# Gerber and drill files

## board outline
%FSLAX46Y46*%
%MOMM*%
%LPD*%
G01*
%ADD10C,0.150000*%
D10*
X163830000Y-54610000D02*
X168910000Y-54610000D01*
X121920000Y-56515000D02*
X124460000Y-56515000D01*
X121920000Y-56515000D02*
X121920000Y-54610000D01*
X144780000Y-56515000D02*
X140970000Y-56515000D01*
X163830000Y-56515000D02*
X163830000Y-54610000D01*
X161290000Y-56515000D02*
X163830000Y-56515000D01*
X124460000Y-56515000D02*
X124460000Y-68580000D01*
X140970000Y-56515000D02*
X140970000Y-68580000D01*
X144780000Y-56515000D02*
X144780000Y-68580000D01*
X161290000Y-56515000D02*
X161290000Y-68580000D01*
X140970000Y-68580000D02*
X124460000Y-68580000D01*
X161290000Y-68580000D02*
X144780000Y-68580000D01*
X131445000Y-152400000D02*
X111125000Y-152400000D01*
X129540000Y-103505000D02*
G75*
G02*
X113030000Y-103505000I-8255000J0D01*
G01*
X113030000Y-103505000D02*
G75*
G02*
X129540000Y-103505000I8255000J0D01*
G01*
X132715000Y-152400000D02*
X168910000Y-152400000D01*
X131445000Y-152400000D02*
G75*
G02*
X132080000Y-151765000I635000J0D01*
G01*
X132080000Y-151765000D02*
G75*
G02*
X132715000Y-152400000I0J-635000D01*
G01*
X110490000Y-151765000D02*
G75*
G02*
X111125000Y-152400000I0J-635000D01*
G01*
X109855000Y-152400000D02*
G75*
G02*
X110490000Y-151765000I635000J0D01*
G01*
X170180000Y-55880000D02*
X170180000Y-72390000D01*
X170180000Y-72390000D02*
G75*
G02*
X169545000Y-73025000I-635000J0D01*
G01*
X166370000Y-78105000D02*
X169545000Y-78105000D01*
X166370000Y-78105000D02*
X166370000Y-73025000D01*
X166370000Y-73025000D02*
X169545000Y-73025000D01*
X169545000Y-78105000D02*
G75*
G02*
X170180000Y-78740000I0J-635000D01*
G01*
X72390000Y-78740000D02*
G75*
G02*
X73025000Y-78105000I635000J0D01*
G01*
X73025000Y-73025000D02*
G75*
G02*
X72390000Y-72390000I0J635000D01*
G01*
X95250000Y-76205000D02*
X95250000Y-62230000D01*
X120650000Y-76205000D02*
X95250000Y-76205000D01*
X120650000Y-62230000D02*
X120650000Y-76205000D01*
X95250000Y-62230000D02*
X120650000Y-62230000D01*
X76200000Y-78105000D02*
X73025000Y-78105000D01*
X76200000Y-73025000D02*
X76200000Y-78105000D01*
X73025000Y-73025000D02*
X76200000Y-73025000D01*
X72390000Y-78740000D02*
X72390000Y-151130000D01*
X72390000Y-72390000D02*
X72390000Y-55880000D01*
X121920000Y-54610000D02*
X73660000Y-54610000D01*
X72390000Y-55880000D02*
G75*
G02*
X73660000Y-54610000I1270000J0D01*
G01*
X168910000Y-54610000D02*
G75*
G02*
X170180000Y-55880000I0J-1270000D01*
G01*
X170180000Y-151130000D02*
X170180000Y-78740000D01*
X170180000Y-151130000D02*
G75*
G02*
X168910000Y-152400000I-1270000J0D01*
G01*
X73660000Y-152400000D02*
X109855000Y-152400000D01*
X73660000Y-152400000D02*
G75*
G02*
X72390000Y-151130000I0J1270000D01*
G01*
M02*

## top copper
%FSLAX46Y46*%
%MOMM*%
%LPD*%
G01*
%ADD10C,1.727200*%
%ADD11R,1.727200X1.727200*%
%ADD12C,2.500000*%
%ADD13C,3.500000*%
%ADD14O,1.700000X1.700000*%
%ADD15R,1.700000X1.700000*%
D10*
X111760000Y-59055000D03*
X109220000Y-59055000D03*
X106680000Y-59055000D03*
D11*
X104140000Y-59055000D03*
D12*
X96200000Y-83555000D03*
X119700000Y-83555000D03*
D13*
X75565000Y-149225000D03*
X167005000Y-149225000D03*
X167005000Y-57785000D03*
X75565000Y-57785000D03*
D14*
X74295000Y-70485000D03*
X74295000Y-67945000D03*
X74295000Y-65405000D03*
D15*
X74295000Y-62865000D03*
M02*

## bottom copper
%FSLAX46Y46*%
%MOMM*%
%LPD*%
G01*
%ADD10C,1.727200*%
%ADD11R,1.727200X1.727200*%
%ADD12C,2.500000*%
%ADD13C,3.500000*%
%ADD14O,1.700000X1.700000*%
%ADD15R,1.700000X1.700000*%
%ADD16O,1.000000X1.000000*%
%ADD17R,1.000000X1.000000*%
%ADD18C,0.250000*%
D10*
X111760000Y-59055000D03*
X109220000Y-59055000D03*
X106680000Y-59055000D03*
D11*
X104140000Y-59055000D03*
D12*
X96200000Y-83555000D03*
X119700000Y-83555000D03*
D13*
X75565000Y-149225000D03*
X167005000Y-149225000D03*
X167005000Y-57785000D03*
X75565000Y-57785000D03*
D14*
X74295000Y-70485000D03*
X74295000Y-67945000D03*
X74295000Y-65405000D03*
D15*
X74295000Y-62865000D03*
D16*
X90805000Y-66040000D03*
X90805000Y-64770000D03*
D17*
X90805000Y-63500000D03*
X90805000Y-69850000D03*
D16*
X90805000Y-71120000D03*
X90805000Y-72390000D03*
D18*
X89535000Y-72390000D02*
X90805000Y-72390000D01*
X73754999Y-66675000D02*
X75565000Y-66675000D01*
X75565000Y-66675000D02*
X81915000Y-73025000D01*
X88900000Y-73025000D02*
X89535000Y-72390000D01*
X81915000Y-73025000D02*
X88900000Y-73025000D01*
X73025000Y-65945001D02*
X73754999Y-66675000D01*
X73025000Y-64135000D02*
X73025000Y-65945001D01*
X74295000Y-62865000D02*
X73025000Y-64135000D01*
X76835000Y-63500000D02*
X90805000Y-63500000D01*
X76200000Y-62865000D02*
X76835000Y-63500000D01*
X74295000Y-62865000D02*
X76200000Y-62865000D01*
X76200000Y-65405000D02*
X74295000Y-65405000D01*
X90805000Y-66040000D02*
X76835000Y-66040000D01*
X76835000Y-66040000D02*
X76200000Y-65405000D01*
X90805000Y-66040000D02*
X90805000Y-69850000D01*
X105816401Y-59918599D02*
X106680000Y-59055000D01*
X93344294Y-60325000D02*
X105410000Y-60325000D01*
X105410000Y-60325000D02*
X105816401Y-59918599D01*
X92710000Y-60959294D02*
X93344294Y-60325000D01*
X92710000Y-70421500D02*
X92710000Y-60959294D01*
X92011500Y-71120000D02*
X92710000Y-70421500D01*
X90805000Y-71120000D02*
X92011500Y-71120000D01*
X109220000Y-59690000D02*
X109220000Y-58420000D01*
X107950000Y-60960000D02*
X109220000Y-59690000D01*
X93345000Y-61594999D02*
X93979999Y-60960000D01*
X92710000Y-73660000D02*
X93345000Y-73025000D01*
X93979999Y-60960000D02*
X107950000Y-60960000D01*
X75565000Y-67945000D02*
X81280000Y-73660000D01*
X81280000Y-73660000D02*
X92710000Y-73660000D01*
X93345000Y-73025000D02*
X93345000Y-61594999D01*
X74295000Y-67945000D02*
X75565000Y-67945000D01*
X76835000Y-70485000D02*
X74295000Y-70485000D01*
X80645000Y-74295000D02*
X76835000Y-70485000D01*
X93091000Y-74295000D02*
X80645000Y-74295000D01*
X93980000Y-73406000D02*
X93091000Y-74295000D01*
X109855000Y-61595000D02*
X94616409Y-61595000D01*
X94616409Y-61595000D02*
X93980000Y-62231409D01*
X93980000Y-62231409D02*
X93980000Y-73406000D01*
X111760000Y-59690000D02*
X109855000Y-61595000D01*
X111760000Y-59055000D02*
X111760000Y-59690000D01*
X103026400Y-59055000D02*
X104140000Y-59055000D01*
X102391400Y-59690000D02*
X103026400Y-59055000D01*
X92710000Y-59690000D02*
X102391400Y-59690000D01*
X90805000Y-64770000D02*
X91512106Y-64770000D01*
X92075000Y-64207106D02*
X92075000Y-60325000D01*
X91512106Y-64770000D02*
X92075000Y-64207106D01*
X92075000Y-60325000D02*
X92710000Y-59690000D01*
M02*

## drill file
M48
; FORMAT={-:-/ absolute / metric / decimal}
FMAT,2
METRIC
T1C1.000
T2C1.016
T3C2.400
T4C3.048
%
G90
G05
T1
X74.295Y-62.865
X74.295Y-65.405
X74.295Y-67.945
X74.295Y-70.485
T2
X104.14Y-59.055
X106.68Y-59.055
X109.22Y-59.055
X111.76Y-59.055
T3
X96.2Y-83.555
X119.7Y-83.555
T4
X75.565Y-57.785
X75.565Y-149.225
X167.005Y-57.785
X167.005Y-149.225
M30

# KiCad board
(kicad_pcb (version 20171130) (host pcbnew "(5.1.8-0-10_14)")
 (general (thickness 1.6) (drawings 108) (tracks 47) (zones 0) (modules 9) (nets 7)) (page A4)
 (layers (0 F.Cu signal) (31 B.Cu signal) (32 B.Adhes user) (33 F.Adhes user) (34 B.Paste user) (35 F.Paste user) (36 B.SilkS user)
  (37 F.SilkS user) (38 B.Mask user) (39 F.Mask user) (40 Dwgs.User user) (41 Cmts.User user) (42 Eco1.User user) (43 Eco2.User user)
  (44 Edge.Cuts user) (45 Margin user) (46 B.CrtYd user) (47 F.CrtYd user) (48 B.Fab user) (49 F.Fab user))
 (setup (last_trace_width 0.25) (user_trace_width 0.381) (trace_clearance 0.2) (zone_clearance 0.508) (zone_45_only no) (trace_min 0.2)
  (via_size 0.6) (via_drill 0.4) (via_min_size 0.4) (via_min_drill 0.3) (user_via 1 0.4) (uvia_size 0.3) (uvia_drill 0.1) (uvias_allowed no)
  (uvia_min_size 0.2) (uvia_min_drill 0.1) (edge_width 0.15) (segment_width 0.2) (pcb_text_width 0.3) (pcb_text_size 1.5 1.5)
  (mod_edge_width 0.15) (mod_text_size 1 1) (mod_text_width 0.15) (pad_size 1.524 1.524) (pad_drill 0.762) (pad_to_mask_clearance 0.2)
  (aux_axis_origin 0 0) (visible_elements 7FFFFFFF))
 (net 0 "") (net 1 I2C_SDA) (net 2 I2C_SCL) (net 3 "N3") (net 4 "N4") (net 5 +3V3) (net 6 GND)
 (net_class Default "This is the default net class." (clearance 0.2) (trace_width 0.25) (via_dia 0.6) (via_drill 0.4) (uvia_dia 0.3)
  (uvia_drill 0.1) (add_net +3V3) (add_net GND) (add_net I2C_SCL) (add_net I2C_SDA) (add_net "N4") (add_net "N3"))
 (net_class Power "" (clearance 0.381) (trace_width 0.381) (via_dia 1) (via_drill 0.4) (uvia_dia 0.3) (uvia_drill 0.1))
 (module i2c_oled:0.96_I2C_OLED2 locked (layer F.Cu) (at 107.95 59.055)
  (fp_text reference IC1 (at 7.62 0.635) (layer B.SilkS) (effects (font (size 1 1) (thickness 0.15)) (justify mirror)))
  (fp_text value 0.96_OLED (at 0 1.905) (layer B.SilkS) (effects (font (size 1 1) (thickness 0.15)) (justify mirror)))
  (pad 4 thru_hole circle (at 3.81 0) (size 1.7272 1.7272) (drill 1.016) (layers *.Cu *.Mask) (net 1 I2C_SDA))
  (pad 3 thru_hole circle (at 1.27 0) (size 1.7272 1.7272) (drill 1.016) (layers *.Cu *.Mask) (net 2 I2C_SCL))
  (pad 2 thru_hole circle (at -1.27 0) (size 1.7272 1.7272) (drill 1.016) (layers *.Cu *.Mask) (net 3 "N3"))
  (pad 1 thru_hole rect (at -3.81 0) (size 1.7272 1.7272) (drill 1.016) (layers *.Cu *.Mask) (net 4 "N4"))
  (pad "" np_thru_hole circle (at -11.75 24.5) (size 2.5 2.5) (drill 2.4) (layers *.Cu *.Mask))
  (pad "" np_thru_hole circle (at 11.75 24.5) (size 2.5 2.5) (drill 2.4) (layers *.Cu *.Mask)))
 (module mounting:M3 (layer F.Cu) (at 75.565 149.225)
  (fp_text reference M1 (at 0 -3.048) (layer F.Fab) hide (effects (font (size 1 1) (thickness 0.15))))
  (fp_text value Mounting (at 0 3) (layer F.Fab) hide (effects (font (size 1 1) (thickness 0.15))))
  (pad "" np_thru_hole circle (at 0 0) (size 3.5 3.5) (drill 3.048) (layers *.Cu *.Mask) (solder_mask_margin 0.8)))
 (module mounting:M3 (layer F.Cu) (at 167.005 149.225)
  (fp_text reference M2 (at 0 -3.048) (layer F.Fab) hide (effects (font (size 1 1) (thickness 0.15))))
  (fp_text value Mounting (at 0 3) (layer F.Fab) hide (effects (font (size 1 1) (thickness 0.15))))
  (pad "" np_thru_hole circle (at 0 0) (size 3.5 3.5) (drill 3.048) (layers *.Cu *.Mask) (solder_mask_margin 0.8)))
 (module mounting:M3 (layer F.Cu) (at 167.005 57.785)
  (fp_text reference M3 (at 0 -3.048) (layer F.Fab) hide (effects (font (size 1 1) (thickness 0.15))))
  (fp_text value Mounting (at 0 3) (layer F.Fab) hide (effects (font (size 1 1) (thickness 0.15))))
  (pad "" np_thru_hole circle (at 0 0) (size 3.5 3.5) (drill 3.048) (layers *.Cu *.Mask) (solder_mask_margin 0.8)))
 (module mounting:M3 (layer F.Cu) (at 75.565 57.785)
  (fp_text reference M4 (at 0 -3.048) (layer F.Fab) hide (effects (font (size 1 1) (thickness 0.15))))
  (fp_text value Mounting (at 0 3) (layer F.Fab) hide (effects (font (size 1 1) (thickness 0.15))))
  (pad "" np_thru_hole circle (at 0 0) (size 3.5 3.5) (drill 3.048) (layers *.Cu *.Mask) (solder_mask_margin 0.8)))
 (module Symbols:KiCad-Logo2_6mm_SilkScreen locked (layer B.Cu) (at 142.875 88.9 180)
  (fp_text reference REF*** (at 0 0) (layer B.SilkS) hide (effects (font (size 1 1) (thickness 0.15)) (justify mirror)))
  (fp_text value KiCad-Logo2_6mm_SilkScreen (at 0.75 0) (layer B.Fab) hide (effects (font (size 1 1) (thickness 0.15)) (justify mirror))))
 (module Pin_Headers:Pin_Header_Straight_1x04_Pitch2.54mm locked (layer B.Cu) (at 74.295 62.865 180)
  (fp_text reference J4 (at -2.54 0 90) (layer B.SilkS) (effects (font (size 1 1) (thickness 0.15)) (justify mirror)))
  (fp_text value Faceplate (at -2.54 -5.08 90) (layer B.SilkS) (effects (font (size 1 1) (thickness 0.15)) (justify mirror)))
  (pad 4 thru_hole oval (at 0 -7.62 180) (size 1.7 1.7) (drill 1) (layers *.Cu *.Mask) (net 1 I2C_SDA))
  (pad 3 thru_hole oval (at 0 -5.08 180) (size 1.7 1.7) (drill 1) (layers *.Cu *.Mask) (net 2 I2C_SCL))
  (pad 2 thru_hole oval (at 0 -2.54 180) (size 1.7 1.7) (drill 1) (layers *.Cu *.Mask) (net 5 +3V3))
  (pad 1 thru_hole rect (at 0 0 180) (size 1.7 1.7) (drill 1) (layers *.Cu *.Mask) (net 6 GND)))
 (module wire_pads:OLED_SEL (layer B.Cu) (at 90.805 63.5 180)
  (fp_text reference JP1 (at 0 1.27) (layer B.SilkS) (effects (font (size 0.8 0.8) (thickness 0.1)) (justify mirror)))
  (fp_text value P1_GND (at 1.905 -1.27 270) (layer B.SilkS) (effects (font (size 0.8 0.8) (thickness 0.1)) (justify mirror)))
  (pad 3 smd oval (at 0 -2.54 180) (size 1 1) (layers B.Cu B.Paste B.Mask) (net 5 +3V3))
  (pad 2 smd oval (at 0 -1.27 180) (size 1 1) (layers B.Cu B.Paste B.Mask) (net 4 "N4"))
  (pad 1 smd rect (at 0 0 180) (size 1 1) (layers B.Cu B.Paste B.Mask) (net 6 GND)))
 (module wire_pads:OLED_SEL (layer B.Cu) (at 90.805 69.85 180)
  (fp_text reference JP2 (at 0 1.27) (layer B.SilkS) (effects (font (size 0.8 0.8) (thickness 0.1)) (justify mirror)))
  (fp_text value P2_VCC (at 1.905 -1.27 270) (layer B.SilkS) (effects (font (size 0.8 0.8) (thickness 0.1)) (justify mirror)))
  (pad 1 smd rect (at 0 0 180) (size 1 1) (layers B.Cu B.Paste B.Mask) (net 5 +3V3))
  (pad 2 smd oval (at 0 -1.27 180) (size 1 1) (layers B.Cu B.Paste B.Mask) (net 3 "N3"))
  (pad 3 smd oval (at 0 -2.54 180) (size 1 1) (layers B.Cu B.Paste B.Mask) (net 6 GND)))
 (gr_line (start 163.83 54.61) (end 168.91 54.61) (layer Edge.Cuts) (width 0.15))
 (gr_line (start 121.92 56.515) (end 124.46 56.515) (layer Edge.Cuts) (width 0.15))
 (gr_line (start 121.92 56.515) (end 121.92 54.61) (layer Edge.Cuts) (width 0.15))
 (gr_line (start 144.78 56.515) (end 140.97 56.515) (layer Edge.Cuts) (width 0.15))
 (gr_line (start 163.83 56.515) (end 163.83 54.61) (layer Edge.Cuts) (width 0.15))
 (gr_line (start 161.29 56.515) (end 163.83 56.515) (layer Edge.Cuts) (width 0.15))
 (gr_line (start 124.46 56.515) (end 124.46 68.58) (layer Edge.Cuts) (width 0.15))
 (gr_line (start 140.97 56.515) (end 140.97 68.58) (layer Edge.Cuts) (width 0.15))
 (gr_line (start 144.78 56.515) (end 144.78 68.58) (layer Edge.Cuts) (width 0.15))
 (gr_line (start 161.29 56.515) (end 161.29 68.58) (layer Edge.Cuts) (width 0.15))
 (gr_line (start 140.97 68.58) (end 124.46 68.58) (layer Edge.Cuts) (width 0.15))
 (gr_line (start 161.29 68.58) (end 144.78 68.58) (layer Edge.Cuts) (width 0.15))
 (gr_line (start 131.445 152.4) (end 111.125 152.4) (layer Edge.Cuts) (width 0.15))
 (gr_circle (center 121.285 103.505) (end 129.54 103.505) (layer Edge.Cuts) (width 0.15))
 (gr_line (start 132.715 152.4) (end 168.91 152.4) (layer Edge.Cuts) (width 0.15))
 (gr_arc (start 132.08 152.4) (end 132.08 151.765) (angle -90) (layer Edge.Cuts) (width 0.15))
 (gr_arc (start 132.08 152.4) (end 132.715 152.4) (angle -90) (layer Edge.Cuts) (width 0.15))
 (gr_arc (start 110.49 152.4) (end 111.125 152.4) (angle -90) (layer Edge.Cuts) (width 0.15))
 (gr_arc (start 110.49 152.4) (end 110.49 151.765) (angle -90) (layer Edge.Cuts) (width 0.15))
 (gr_line (start 170.18 55.88) (end 170.18 72.39) (layer Edge.Cuts) (width 0.15))
 (gr_arc (start 169.545 72.39) (end 169.545 73.025) (angle -90) (layer Edge.Cuts) (width 0.15))
 (gr_line (start 166.37 78.105) (end 169.545 78.105) (layer Edge.Cuts) (width 0.15))
 (gr_line (start 166.37 78.105) (end 166.37 73.025) (layer Edge.Cuts) (width 0.15))
 (gr_line (start 166.37 73.025) (end 169.545 73.025) (layer Edge.Cuts) (width 0.15))
 (gr_arc (start 169.545 78.74) (end 170.18 78.74) (angle -90) (layer Edge.Cuts) (width 0.15))
 (gr_arc (start 73.025 78.74) (end 73.025 78.105) (angle -90) (layer Edge.Cuts) (width 0.15))
 (gr_arc (start 73.025 72.39) (end 72.39 72.39) (angle -90) (layer Edge.Cuts) (width 0.15))
 (gr_line (start 95.25 76.205) (end 95.25 62.23) (layer Edge.Cuts) (width 0.15))
 (gr_line (start 120.65 76.205) (end 95.25 76.205) (layer Edge.Cuts) (width 0.15))
 (gr_line (start 120.65 62.23) (end 120.65 76.205) (layer Edge.Cuts) (width 0.15))
 (gr_line (start 95.25 62.23) (end 120.65 62.23) (layer Edge.Cuts) (width 0.15))
 (gr_line (start 76.2 78.105) (end 73.025 78.105) (layer Edge.Cuts) (width 0.15))
 (gr_line (start 76.2 73.025) (end 76.2 78.105) (layer Edge.Cuts) (width 0.15))
 (gr_line (start 73.025 73.025) (end 76.2 73.025) (layer Edge.Cuts) (width 0.15))
 (gr_line (start 72.39 78.74) (end 72.39 151.13) (layer Edge.Cuts) (width 0.15))
 (gr_line (start 72.39 72.39) (end 72.39 55.88) (layer Edge.Cuts) (width 0.15))
 (gr_line (start 121.92 54.61) (end 73.66 54.61) (angle 90) (layer Edge.Cuts) (width 0.15))
 (gr_arc (start 73.66 55.88) (end 72.39 55.88) (angle 90) (layer Edge.Cuts) (width 0.15))
 (gr_arc (start 168.91 55.88) (end 168.91 54.61) (angle 90) (layer Edge.Cuts) (width 0.15))
 (gr_line (start 170.18 151.13) (end 170.18 78.74) (angle 90) (layer Edge.Cuts) (width 0.15))
 (gr_arc (start 168.91 151.13) (end 170.18 151.13) (angle 90) (layer Edge.Cuts) (width 0.15))
 (gr_line (start 73.66 152.4) (end 109.855 152.4) (angle 90) (layer Edge.Cuts) (width 0.15))
 (gr_arc (start 73.66 151.13) (end 73.66 152.4) (angle 90) (layer Edge.Cuts) (width 0.15))
 (segment (start 89.535 72.39) (end 90.805 72.39) (width 0.25) (layer B.Cu) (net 6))
 (segment (start 73.754999 66.675) (end 75.565 66.675) (width 0.25) (layer B.Cu) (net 6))
 (segment (start 75.565 66.675) (end 81.915 73.025) (width 0.25) (layer B.Cu) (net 6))
 (segment (start 88.9 73.025) (end 89.535 72.39) (width 0.25) (layer B.Cu) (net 6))
 (segment (start 81.915 73.025) (end 88.9 73.025) (width 0.25) (layer B.Cu) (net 6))
 (segment (start 73.025 65.945001) (end 73.754999 66.675) (width 0.25) (layer B.Cu) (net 6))
 (segment (start 73.025 64.135) (end 73.025 65.945001) (width 0.25) (layer B.Cu) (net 6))
 (segment (start 74.295 62.865) (end 73.025 64.135) (width 0.25) (layer B.Cu) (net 6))
 (segment (start 76.835 63.5) (end 90.805 63.5) (width 0.25) (layer B.Cu) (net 6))
 (segment (start 76.2 62.865) (end 76.835 63.5) (width 0.25) (layer B.Cu) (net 6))
 (segment (start 74.295 62.865) (end 76.2 62.865) (width 0.25) (layer B.Cu) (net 6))
 (segment (start 76.2 65.405) (end 74.295 65.405) (width 0.25) (layer B.Cu) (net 5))
 (segment (start 90.805 66.04) (end 76.835 66.04) (width 0.25) (layer B.Cu) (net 5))
 (segment (start 76.835 66.04) (end 76.2 65.405) (width 0.25) (layer B.Cu) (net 5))
 (segment (start 90.805 66.04) (end 90.805 69.85) (width 0.25) (layer B.Cu) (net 5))
 (segment (start 105.816401 59.918599) (end 106.68 59.055) (width 0.25) (layer B.Cu) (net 3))
 (segment (start 93.344294 60.325) (end 105.41 60.325) (width 0.25) (layer B.Cu) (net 3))
 (segment (start 105.41 60.325) (end 105.816401 59.918599) (width 0.25) (layer B.Cu) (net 3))
 (segment (start 92.71 60.959294) (end 93.344294 60.325) (width 0.25) (layer B.Cu) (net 3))
 (segment (start 92.71 70.4215) (end 92.71 60.959294) (width 0.25) (layer B.Cu) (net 3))
 (segment (start 92.0115 71.12) (end 92.71 70.4215) (width 0.25) (layer B.Cu) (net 3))
 (segment (start 90.805 71.12) (end 92.0115 71.12) (width 0.25) (layer B.Cu) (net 3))
 (segment (start 109.22 59.69) (end 109.22 58.42) (width 0.25) (layer B.Cu) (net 2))
 (segment (start 107.95 60.96) (end 109.22 59.69) (width 0.25) (layer B.Cu) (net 2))
 (segment (start 93.345 61.594999) (end 93.979999 60.96) (width 0.25) (layer B.Cu) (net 2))
 (segment (start 92.71 73.66) (end 93.345 73.025) (width 0.25) (layer B.Cu) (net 2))
 (segment (start 93.979999 60.96) (end 107.95 60.96) (width 0.25) (layer B.Cu) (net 2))
 (segment (start 75.565 67.945) (end 81.28 73.66) (width 0.25) (layer B.Cu) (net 2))
 (segment (start 81.28 73.66) (end 92.71 73.66) (width 0.25) (layer B.Cu) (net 2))
 (segment (start 93.345 73.025) (end 93.345 61.594999) (width 0.25) (layer B.Cu) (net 2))
 (segment (start 74.295 67.945) (end 75.565 67.945) (width 0.25) (layer B.Cu) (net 2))
 (segment (start 76.835 70.485) (end 74.295 70.485) (width 0.25) (layer B.Cu) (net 1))
 (segment (start 80.645 74.295) (end 76.835 70.485) (width 0.25) (layer B.Cu) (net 1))
 (segment (start 93.091 74.295) (end 80.645 74.295) (width 0.25) (layer B.Cu) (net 1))
 (segment (start 93.98 73.406) (end 93.091 74.295) (width 0.25) (layer B.Cu) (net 1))
 (segment (start 109.855 61.595) (end 94.616409 61.595) (width 0.25) (layer B.Cu) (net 1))
 (segment (start 94.616409 61.595) (end 93.98 62.231409) (width 0.25) (layer B.Cu) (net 1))
 (segment (start 93.98 62.231409) (end 93.98 73.406) (width 0.25) (layer B.Cu) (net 1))
 (segment (start 111.76 59.69) (end 109.855 61.595) (width 0.25) (layer B.Cu) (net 1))
 (segment (start 111.76 59.055) (end 111.76 59.69) (width 0.25) (layer B.Cu) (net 1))
 (segment (start 103.0264 59.055) (end 104.14 59.055) (width 0.25) (layer B.Cu) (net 4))
 (segment (start 102.3914 59.69) (end 103.0264 59.055) (width 0.25) (layer B.Cu) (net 4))
 (segment (start 92.71 59.69) (end 102.3914 59.69) (width 0.25) (layer B.Cu) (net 4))
 (segment (start 90.805 64.77) (end 91.512106 64.77) (width 0.25) (layer B.Cu) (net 4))
 (segment (start 92.075 64.207106) (end 92.075 60.325) (width 0.25) (layer B.Cu) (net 4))
 (segment (start 91.512106 64.77) (end 92.075 64.207106) (width 0.25) (layer B.Cu) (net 4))
 (segment (start 92.075 60.325) (end 92.71 59.69) (width 0.25) (layer B.Cu) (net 4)))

